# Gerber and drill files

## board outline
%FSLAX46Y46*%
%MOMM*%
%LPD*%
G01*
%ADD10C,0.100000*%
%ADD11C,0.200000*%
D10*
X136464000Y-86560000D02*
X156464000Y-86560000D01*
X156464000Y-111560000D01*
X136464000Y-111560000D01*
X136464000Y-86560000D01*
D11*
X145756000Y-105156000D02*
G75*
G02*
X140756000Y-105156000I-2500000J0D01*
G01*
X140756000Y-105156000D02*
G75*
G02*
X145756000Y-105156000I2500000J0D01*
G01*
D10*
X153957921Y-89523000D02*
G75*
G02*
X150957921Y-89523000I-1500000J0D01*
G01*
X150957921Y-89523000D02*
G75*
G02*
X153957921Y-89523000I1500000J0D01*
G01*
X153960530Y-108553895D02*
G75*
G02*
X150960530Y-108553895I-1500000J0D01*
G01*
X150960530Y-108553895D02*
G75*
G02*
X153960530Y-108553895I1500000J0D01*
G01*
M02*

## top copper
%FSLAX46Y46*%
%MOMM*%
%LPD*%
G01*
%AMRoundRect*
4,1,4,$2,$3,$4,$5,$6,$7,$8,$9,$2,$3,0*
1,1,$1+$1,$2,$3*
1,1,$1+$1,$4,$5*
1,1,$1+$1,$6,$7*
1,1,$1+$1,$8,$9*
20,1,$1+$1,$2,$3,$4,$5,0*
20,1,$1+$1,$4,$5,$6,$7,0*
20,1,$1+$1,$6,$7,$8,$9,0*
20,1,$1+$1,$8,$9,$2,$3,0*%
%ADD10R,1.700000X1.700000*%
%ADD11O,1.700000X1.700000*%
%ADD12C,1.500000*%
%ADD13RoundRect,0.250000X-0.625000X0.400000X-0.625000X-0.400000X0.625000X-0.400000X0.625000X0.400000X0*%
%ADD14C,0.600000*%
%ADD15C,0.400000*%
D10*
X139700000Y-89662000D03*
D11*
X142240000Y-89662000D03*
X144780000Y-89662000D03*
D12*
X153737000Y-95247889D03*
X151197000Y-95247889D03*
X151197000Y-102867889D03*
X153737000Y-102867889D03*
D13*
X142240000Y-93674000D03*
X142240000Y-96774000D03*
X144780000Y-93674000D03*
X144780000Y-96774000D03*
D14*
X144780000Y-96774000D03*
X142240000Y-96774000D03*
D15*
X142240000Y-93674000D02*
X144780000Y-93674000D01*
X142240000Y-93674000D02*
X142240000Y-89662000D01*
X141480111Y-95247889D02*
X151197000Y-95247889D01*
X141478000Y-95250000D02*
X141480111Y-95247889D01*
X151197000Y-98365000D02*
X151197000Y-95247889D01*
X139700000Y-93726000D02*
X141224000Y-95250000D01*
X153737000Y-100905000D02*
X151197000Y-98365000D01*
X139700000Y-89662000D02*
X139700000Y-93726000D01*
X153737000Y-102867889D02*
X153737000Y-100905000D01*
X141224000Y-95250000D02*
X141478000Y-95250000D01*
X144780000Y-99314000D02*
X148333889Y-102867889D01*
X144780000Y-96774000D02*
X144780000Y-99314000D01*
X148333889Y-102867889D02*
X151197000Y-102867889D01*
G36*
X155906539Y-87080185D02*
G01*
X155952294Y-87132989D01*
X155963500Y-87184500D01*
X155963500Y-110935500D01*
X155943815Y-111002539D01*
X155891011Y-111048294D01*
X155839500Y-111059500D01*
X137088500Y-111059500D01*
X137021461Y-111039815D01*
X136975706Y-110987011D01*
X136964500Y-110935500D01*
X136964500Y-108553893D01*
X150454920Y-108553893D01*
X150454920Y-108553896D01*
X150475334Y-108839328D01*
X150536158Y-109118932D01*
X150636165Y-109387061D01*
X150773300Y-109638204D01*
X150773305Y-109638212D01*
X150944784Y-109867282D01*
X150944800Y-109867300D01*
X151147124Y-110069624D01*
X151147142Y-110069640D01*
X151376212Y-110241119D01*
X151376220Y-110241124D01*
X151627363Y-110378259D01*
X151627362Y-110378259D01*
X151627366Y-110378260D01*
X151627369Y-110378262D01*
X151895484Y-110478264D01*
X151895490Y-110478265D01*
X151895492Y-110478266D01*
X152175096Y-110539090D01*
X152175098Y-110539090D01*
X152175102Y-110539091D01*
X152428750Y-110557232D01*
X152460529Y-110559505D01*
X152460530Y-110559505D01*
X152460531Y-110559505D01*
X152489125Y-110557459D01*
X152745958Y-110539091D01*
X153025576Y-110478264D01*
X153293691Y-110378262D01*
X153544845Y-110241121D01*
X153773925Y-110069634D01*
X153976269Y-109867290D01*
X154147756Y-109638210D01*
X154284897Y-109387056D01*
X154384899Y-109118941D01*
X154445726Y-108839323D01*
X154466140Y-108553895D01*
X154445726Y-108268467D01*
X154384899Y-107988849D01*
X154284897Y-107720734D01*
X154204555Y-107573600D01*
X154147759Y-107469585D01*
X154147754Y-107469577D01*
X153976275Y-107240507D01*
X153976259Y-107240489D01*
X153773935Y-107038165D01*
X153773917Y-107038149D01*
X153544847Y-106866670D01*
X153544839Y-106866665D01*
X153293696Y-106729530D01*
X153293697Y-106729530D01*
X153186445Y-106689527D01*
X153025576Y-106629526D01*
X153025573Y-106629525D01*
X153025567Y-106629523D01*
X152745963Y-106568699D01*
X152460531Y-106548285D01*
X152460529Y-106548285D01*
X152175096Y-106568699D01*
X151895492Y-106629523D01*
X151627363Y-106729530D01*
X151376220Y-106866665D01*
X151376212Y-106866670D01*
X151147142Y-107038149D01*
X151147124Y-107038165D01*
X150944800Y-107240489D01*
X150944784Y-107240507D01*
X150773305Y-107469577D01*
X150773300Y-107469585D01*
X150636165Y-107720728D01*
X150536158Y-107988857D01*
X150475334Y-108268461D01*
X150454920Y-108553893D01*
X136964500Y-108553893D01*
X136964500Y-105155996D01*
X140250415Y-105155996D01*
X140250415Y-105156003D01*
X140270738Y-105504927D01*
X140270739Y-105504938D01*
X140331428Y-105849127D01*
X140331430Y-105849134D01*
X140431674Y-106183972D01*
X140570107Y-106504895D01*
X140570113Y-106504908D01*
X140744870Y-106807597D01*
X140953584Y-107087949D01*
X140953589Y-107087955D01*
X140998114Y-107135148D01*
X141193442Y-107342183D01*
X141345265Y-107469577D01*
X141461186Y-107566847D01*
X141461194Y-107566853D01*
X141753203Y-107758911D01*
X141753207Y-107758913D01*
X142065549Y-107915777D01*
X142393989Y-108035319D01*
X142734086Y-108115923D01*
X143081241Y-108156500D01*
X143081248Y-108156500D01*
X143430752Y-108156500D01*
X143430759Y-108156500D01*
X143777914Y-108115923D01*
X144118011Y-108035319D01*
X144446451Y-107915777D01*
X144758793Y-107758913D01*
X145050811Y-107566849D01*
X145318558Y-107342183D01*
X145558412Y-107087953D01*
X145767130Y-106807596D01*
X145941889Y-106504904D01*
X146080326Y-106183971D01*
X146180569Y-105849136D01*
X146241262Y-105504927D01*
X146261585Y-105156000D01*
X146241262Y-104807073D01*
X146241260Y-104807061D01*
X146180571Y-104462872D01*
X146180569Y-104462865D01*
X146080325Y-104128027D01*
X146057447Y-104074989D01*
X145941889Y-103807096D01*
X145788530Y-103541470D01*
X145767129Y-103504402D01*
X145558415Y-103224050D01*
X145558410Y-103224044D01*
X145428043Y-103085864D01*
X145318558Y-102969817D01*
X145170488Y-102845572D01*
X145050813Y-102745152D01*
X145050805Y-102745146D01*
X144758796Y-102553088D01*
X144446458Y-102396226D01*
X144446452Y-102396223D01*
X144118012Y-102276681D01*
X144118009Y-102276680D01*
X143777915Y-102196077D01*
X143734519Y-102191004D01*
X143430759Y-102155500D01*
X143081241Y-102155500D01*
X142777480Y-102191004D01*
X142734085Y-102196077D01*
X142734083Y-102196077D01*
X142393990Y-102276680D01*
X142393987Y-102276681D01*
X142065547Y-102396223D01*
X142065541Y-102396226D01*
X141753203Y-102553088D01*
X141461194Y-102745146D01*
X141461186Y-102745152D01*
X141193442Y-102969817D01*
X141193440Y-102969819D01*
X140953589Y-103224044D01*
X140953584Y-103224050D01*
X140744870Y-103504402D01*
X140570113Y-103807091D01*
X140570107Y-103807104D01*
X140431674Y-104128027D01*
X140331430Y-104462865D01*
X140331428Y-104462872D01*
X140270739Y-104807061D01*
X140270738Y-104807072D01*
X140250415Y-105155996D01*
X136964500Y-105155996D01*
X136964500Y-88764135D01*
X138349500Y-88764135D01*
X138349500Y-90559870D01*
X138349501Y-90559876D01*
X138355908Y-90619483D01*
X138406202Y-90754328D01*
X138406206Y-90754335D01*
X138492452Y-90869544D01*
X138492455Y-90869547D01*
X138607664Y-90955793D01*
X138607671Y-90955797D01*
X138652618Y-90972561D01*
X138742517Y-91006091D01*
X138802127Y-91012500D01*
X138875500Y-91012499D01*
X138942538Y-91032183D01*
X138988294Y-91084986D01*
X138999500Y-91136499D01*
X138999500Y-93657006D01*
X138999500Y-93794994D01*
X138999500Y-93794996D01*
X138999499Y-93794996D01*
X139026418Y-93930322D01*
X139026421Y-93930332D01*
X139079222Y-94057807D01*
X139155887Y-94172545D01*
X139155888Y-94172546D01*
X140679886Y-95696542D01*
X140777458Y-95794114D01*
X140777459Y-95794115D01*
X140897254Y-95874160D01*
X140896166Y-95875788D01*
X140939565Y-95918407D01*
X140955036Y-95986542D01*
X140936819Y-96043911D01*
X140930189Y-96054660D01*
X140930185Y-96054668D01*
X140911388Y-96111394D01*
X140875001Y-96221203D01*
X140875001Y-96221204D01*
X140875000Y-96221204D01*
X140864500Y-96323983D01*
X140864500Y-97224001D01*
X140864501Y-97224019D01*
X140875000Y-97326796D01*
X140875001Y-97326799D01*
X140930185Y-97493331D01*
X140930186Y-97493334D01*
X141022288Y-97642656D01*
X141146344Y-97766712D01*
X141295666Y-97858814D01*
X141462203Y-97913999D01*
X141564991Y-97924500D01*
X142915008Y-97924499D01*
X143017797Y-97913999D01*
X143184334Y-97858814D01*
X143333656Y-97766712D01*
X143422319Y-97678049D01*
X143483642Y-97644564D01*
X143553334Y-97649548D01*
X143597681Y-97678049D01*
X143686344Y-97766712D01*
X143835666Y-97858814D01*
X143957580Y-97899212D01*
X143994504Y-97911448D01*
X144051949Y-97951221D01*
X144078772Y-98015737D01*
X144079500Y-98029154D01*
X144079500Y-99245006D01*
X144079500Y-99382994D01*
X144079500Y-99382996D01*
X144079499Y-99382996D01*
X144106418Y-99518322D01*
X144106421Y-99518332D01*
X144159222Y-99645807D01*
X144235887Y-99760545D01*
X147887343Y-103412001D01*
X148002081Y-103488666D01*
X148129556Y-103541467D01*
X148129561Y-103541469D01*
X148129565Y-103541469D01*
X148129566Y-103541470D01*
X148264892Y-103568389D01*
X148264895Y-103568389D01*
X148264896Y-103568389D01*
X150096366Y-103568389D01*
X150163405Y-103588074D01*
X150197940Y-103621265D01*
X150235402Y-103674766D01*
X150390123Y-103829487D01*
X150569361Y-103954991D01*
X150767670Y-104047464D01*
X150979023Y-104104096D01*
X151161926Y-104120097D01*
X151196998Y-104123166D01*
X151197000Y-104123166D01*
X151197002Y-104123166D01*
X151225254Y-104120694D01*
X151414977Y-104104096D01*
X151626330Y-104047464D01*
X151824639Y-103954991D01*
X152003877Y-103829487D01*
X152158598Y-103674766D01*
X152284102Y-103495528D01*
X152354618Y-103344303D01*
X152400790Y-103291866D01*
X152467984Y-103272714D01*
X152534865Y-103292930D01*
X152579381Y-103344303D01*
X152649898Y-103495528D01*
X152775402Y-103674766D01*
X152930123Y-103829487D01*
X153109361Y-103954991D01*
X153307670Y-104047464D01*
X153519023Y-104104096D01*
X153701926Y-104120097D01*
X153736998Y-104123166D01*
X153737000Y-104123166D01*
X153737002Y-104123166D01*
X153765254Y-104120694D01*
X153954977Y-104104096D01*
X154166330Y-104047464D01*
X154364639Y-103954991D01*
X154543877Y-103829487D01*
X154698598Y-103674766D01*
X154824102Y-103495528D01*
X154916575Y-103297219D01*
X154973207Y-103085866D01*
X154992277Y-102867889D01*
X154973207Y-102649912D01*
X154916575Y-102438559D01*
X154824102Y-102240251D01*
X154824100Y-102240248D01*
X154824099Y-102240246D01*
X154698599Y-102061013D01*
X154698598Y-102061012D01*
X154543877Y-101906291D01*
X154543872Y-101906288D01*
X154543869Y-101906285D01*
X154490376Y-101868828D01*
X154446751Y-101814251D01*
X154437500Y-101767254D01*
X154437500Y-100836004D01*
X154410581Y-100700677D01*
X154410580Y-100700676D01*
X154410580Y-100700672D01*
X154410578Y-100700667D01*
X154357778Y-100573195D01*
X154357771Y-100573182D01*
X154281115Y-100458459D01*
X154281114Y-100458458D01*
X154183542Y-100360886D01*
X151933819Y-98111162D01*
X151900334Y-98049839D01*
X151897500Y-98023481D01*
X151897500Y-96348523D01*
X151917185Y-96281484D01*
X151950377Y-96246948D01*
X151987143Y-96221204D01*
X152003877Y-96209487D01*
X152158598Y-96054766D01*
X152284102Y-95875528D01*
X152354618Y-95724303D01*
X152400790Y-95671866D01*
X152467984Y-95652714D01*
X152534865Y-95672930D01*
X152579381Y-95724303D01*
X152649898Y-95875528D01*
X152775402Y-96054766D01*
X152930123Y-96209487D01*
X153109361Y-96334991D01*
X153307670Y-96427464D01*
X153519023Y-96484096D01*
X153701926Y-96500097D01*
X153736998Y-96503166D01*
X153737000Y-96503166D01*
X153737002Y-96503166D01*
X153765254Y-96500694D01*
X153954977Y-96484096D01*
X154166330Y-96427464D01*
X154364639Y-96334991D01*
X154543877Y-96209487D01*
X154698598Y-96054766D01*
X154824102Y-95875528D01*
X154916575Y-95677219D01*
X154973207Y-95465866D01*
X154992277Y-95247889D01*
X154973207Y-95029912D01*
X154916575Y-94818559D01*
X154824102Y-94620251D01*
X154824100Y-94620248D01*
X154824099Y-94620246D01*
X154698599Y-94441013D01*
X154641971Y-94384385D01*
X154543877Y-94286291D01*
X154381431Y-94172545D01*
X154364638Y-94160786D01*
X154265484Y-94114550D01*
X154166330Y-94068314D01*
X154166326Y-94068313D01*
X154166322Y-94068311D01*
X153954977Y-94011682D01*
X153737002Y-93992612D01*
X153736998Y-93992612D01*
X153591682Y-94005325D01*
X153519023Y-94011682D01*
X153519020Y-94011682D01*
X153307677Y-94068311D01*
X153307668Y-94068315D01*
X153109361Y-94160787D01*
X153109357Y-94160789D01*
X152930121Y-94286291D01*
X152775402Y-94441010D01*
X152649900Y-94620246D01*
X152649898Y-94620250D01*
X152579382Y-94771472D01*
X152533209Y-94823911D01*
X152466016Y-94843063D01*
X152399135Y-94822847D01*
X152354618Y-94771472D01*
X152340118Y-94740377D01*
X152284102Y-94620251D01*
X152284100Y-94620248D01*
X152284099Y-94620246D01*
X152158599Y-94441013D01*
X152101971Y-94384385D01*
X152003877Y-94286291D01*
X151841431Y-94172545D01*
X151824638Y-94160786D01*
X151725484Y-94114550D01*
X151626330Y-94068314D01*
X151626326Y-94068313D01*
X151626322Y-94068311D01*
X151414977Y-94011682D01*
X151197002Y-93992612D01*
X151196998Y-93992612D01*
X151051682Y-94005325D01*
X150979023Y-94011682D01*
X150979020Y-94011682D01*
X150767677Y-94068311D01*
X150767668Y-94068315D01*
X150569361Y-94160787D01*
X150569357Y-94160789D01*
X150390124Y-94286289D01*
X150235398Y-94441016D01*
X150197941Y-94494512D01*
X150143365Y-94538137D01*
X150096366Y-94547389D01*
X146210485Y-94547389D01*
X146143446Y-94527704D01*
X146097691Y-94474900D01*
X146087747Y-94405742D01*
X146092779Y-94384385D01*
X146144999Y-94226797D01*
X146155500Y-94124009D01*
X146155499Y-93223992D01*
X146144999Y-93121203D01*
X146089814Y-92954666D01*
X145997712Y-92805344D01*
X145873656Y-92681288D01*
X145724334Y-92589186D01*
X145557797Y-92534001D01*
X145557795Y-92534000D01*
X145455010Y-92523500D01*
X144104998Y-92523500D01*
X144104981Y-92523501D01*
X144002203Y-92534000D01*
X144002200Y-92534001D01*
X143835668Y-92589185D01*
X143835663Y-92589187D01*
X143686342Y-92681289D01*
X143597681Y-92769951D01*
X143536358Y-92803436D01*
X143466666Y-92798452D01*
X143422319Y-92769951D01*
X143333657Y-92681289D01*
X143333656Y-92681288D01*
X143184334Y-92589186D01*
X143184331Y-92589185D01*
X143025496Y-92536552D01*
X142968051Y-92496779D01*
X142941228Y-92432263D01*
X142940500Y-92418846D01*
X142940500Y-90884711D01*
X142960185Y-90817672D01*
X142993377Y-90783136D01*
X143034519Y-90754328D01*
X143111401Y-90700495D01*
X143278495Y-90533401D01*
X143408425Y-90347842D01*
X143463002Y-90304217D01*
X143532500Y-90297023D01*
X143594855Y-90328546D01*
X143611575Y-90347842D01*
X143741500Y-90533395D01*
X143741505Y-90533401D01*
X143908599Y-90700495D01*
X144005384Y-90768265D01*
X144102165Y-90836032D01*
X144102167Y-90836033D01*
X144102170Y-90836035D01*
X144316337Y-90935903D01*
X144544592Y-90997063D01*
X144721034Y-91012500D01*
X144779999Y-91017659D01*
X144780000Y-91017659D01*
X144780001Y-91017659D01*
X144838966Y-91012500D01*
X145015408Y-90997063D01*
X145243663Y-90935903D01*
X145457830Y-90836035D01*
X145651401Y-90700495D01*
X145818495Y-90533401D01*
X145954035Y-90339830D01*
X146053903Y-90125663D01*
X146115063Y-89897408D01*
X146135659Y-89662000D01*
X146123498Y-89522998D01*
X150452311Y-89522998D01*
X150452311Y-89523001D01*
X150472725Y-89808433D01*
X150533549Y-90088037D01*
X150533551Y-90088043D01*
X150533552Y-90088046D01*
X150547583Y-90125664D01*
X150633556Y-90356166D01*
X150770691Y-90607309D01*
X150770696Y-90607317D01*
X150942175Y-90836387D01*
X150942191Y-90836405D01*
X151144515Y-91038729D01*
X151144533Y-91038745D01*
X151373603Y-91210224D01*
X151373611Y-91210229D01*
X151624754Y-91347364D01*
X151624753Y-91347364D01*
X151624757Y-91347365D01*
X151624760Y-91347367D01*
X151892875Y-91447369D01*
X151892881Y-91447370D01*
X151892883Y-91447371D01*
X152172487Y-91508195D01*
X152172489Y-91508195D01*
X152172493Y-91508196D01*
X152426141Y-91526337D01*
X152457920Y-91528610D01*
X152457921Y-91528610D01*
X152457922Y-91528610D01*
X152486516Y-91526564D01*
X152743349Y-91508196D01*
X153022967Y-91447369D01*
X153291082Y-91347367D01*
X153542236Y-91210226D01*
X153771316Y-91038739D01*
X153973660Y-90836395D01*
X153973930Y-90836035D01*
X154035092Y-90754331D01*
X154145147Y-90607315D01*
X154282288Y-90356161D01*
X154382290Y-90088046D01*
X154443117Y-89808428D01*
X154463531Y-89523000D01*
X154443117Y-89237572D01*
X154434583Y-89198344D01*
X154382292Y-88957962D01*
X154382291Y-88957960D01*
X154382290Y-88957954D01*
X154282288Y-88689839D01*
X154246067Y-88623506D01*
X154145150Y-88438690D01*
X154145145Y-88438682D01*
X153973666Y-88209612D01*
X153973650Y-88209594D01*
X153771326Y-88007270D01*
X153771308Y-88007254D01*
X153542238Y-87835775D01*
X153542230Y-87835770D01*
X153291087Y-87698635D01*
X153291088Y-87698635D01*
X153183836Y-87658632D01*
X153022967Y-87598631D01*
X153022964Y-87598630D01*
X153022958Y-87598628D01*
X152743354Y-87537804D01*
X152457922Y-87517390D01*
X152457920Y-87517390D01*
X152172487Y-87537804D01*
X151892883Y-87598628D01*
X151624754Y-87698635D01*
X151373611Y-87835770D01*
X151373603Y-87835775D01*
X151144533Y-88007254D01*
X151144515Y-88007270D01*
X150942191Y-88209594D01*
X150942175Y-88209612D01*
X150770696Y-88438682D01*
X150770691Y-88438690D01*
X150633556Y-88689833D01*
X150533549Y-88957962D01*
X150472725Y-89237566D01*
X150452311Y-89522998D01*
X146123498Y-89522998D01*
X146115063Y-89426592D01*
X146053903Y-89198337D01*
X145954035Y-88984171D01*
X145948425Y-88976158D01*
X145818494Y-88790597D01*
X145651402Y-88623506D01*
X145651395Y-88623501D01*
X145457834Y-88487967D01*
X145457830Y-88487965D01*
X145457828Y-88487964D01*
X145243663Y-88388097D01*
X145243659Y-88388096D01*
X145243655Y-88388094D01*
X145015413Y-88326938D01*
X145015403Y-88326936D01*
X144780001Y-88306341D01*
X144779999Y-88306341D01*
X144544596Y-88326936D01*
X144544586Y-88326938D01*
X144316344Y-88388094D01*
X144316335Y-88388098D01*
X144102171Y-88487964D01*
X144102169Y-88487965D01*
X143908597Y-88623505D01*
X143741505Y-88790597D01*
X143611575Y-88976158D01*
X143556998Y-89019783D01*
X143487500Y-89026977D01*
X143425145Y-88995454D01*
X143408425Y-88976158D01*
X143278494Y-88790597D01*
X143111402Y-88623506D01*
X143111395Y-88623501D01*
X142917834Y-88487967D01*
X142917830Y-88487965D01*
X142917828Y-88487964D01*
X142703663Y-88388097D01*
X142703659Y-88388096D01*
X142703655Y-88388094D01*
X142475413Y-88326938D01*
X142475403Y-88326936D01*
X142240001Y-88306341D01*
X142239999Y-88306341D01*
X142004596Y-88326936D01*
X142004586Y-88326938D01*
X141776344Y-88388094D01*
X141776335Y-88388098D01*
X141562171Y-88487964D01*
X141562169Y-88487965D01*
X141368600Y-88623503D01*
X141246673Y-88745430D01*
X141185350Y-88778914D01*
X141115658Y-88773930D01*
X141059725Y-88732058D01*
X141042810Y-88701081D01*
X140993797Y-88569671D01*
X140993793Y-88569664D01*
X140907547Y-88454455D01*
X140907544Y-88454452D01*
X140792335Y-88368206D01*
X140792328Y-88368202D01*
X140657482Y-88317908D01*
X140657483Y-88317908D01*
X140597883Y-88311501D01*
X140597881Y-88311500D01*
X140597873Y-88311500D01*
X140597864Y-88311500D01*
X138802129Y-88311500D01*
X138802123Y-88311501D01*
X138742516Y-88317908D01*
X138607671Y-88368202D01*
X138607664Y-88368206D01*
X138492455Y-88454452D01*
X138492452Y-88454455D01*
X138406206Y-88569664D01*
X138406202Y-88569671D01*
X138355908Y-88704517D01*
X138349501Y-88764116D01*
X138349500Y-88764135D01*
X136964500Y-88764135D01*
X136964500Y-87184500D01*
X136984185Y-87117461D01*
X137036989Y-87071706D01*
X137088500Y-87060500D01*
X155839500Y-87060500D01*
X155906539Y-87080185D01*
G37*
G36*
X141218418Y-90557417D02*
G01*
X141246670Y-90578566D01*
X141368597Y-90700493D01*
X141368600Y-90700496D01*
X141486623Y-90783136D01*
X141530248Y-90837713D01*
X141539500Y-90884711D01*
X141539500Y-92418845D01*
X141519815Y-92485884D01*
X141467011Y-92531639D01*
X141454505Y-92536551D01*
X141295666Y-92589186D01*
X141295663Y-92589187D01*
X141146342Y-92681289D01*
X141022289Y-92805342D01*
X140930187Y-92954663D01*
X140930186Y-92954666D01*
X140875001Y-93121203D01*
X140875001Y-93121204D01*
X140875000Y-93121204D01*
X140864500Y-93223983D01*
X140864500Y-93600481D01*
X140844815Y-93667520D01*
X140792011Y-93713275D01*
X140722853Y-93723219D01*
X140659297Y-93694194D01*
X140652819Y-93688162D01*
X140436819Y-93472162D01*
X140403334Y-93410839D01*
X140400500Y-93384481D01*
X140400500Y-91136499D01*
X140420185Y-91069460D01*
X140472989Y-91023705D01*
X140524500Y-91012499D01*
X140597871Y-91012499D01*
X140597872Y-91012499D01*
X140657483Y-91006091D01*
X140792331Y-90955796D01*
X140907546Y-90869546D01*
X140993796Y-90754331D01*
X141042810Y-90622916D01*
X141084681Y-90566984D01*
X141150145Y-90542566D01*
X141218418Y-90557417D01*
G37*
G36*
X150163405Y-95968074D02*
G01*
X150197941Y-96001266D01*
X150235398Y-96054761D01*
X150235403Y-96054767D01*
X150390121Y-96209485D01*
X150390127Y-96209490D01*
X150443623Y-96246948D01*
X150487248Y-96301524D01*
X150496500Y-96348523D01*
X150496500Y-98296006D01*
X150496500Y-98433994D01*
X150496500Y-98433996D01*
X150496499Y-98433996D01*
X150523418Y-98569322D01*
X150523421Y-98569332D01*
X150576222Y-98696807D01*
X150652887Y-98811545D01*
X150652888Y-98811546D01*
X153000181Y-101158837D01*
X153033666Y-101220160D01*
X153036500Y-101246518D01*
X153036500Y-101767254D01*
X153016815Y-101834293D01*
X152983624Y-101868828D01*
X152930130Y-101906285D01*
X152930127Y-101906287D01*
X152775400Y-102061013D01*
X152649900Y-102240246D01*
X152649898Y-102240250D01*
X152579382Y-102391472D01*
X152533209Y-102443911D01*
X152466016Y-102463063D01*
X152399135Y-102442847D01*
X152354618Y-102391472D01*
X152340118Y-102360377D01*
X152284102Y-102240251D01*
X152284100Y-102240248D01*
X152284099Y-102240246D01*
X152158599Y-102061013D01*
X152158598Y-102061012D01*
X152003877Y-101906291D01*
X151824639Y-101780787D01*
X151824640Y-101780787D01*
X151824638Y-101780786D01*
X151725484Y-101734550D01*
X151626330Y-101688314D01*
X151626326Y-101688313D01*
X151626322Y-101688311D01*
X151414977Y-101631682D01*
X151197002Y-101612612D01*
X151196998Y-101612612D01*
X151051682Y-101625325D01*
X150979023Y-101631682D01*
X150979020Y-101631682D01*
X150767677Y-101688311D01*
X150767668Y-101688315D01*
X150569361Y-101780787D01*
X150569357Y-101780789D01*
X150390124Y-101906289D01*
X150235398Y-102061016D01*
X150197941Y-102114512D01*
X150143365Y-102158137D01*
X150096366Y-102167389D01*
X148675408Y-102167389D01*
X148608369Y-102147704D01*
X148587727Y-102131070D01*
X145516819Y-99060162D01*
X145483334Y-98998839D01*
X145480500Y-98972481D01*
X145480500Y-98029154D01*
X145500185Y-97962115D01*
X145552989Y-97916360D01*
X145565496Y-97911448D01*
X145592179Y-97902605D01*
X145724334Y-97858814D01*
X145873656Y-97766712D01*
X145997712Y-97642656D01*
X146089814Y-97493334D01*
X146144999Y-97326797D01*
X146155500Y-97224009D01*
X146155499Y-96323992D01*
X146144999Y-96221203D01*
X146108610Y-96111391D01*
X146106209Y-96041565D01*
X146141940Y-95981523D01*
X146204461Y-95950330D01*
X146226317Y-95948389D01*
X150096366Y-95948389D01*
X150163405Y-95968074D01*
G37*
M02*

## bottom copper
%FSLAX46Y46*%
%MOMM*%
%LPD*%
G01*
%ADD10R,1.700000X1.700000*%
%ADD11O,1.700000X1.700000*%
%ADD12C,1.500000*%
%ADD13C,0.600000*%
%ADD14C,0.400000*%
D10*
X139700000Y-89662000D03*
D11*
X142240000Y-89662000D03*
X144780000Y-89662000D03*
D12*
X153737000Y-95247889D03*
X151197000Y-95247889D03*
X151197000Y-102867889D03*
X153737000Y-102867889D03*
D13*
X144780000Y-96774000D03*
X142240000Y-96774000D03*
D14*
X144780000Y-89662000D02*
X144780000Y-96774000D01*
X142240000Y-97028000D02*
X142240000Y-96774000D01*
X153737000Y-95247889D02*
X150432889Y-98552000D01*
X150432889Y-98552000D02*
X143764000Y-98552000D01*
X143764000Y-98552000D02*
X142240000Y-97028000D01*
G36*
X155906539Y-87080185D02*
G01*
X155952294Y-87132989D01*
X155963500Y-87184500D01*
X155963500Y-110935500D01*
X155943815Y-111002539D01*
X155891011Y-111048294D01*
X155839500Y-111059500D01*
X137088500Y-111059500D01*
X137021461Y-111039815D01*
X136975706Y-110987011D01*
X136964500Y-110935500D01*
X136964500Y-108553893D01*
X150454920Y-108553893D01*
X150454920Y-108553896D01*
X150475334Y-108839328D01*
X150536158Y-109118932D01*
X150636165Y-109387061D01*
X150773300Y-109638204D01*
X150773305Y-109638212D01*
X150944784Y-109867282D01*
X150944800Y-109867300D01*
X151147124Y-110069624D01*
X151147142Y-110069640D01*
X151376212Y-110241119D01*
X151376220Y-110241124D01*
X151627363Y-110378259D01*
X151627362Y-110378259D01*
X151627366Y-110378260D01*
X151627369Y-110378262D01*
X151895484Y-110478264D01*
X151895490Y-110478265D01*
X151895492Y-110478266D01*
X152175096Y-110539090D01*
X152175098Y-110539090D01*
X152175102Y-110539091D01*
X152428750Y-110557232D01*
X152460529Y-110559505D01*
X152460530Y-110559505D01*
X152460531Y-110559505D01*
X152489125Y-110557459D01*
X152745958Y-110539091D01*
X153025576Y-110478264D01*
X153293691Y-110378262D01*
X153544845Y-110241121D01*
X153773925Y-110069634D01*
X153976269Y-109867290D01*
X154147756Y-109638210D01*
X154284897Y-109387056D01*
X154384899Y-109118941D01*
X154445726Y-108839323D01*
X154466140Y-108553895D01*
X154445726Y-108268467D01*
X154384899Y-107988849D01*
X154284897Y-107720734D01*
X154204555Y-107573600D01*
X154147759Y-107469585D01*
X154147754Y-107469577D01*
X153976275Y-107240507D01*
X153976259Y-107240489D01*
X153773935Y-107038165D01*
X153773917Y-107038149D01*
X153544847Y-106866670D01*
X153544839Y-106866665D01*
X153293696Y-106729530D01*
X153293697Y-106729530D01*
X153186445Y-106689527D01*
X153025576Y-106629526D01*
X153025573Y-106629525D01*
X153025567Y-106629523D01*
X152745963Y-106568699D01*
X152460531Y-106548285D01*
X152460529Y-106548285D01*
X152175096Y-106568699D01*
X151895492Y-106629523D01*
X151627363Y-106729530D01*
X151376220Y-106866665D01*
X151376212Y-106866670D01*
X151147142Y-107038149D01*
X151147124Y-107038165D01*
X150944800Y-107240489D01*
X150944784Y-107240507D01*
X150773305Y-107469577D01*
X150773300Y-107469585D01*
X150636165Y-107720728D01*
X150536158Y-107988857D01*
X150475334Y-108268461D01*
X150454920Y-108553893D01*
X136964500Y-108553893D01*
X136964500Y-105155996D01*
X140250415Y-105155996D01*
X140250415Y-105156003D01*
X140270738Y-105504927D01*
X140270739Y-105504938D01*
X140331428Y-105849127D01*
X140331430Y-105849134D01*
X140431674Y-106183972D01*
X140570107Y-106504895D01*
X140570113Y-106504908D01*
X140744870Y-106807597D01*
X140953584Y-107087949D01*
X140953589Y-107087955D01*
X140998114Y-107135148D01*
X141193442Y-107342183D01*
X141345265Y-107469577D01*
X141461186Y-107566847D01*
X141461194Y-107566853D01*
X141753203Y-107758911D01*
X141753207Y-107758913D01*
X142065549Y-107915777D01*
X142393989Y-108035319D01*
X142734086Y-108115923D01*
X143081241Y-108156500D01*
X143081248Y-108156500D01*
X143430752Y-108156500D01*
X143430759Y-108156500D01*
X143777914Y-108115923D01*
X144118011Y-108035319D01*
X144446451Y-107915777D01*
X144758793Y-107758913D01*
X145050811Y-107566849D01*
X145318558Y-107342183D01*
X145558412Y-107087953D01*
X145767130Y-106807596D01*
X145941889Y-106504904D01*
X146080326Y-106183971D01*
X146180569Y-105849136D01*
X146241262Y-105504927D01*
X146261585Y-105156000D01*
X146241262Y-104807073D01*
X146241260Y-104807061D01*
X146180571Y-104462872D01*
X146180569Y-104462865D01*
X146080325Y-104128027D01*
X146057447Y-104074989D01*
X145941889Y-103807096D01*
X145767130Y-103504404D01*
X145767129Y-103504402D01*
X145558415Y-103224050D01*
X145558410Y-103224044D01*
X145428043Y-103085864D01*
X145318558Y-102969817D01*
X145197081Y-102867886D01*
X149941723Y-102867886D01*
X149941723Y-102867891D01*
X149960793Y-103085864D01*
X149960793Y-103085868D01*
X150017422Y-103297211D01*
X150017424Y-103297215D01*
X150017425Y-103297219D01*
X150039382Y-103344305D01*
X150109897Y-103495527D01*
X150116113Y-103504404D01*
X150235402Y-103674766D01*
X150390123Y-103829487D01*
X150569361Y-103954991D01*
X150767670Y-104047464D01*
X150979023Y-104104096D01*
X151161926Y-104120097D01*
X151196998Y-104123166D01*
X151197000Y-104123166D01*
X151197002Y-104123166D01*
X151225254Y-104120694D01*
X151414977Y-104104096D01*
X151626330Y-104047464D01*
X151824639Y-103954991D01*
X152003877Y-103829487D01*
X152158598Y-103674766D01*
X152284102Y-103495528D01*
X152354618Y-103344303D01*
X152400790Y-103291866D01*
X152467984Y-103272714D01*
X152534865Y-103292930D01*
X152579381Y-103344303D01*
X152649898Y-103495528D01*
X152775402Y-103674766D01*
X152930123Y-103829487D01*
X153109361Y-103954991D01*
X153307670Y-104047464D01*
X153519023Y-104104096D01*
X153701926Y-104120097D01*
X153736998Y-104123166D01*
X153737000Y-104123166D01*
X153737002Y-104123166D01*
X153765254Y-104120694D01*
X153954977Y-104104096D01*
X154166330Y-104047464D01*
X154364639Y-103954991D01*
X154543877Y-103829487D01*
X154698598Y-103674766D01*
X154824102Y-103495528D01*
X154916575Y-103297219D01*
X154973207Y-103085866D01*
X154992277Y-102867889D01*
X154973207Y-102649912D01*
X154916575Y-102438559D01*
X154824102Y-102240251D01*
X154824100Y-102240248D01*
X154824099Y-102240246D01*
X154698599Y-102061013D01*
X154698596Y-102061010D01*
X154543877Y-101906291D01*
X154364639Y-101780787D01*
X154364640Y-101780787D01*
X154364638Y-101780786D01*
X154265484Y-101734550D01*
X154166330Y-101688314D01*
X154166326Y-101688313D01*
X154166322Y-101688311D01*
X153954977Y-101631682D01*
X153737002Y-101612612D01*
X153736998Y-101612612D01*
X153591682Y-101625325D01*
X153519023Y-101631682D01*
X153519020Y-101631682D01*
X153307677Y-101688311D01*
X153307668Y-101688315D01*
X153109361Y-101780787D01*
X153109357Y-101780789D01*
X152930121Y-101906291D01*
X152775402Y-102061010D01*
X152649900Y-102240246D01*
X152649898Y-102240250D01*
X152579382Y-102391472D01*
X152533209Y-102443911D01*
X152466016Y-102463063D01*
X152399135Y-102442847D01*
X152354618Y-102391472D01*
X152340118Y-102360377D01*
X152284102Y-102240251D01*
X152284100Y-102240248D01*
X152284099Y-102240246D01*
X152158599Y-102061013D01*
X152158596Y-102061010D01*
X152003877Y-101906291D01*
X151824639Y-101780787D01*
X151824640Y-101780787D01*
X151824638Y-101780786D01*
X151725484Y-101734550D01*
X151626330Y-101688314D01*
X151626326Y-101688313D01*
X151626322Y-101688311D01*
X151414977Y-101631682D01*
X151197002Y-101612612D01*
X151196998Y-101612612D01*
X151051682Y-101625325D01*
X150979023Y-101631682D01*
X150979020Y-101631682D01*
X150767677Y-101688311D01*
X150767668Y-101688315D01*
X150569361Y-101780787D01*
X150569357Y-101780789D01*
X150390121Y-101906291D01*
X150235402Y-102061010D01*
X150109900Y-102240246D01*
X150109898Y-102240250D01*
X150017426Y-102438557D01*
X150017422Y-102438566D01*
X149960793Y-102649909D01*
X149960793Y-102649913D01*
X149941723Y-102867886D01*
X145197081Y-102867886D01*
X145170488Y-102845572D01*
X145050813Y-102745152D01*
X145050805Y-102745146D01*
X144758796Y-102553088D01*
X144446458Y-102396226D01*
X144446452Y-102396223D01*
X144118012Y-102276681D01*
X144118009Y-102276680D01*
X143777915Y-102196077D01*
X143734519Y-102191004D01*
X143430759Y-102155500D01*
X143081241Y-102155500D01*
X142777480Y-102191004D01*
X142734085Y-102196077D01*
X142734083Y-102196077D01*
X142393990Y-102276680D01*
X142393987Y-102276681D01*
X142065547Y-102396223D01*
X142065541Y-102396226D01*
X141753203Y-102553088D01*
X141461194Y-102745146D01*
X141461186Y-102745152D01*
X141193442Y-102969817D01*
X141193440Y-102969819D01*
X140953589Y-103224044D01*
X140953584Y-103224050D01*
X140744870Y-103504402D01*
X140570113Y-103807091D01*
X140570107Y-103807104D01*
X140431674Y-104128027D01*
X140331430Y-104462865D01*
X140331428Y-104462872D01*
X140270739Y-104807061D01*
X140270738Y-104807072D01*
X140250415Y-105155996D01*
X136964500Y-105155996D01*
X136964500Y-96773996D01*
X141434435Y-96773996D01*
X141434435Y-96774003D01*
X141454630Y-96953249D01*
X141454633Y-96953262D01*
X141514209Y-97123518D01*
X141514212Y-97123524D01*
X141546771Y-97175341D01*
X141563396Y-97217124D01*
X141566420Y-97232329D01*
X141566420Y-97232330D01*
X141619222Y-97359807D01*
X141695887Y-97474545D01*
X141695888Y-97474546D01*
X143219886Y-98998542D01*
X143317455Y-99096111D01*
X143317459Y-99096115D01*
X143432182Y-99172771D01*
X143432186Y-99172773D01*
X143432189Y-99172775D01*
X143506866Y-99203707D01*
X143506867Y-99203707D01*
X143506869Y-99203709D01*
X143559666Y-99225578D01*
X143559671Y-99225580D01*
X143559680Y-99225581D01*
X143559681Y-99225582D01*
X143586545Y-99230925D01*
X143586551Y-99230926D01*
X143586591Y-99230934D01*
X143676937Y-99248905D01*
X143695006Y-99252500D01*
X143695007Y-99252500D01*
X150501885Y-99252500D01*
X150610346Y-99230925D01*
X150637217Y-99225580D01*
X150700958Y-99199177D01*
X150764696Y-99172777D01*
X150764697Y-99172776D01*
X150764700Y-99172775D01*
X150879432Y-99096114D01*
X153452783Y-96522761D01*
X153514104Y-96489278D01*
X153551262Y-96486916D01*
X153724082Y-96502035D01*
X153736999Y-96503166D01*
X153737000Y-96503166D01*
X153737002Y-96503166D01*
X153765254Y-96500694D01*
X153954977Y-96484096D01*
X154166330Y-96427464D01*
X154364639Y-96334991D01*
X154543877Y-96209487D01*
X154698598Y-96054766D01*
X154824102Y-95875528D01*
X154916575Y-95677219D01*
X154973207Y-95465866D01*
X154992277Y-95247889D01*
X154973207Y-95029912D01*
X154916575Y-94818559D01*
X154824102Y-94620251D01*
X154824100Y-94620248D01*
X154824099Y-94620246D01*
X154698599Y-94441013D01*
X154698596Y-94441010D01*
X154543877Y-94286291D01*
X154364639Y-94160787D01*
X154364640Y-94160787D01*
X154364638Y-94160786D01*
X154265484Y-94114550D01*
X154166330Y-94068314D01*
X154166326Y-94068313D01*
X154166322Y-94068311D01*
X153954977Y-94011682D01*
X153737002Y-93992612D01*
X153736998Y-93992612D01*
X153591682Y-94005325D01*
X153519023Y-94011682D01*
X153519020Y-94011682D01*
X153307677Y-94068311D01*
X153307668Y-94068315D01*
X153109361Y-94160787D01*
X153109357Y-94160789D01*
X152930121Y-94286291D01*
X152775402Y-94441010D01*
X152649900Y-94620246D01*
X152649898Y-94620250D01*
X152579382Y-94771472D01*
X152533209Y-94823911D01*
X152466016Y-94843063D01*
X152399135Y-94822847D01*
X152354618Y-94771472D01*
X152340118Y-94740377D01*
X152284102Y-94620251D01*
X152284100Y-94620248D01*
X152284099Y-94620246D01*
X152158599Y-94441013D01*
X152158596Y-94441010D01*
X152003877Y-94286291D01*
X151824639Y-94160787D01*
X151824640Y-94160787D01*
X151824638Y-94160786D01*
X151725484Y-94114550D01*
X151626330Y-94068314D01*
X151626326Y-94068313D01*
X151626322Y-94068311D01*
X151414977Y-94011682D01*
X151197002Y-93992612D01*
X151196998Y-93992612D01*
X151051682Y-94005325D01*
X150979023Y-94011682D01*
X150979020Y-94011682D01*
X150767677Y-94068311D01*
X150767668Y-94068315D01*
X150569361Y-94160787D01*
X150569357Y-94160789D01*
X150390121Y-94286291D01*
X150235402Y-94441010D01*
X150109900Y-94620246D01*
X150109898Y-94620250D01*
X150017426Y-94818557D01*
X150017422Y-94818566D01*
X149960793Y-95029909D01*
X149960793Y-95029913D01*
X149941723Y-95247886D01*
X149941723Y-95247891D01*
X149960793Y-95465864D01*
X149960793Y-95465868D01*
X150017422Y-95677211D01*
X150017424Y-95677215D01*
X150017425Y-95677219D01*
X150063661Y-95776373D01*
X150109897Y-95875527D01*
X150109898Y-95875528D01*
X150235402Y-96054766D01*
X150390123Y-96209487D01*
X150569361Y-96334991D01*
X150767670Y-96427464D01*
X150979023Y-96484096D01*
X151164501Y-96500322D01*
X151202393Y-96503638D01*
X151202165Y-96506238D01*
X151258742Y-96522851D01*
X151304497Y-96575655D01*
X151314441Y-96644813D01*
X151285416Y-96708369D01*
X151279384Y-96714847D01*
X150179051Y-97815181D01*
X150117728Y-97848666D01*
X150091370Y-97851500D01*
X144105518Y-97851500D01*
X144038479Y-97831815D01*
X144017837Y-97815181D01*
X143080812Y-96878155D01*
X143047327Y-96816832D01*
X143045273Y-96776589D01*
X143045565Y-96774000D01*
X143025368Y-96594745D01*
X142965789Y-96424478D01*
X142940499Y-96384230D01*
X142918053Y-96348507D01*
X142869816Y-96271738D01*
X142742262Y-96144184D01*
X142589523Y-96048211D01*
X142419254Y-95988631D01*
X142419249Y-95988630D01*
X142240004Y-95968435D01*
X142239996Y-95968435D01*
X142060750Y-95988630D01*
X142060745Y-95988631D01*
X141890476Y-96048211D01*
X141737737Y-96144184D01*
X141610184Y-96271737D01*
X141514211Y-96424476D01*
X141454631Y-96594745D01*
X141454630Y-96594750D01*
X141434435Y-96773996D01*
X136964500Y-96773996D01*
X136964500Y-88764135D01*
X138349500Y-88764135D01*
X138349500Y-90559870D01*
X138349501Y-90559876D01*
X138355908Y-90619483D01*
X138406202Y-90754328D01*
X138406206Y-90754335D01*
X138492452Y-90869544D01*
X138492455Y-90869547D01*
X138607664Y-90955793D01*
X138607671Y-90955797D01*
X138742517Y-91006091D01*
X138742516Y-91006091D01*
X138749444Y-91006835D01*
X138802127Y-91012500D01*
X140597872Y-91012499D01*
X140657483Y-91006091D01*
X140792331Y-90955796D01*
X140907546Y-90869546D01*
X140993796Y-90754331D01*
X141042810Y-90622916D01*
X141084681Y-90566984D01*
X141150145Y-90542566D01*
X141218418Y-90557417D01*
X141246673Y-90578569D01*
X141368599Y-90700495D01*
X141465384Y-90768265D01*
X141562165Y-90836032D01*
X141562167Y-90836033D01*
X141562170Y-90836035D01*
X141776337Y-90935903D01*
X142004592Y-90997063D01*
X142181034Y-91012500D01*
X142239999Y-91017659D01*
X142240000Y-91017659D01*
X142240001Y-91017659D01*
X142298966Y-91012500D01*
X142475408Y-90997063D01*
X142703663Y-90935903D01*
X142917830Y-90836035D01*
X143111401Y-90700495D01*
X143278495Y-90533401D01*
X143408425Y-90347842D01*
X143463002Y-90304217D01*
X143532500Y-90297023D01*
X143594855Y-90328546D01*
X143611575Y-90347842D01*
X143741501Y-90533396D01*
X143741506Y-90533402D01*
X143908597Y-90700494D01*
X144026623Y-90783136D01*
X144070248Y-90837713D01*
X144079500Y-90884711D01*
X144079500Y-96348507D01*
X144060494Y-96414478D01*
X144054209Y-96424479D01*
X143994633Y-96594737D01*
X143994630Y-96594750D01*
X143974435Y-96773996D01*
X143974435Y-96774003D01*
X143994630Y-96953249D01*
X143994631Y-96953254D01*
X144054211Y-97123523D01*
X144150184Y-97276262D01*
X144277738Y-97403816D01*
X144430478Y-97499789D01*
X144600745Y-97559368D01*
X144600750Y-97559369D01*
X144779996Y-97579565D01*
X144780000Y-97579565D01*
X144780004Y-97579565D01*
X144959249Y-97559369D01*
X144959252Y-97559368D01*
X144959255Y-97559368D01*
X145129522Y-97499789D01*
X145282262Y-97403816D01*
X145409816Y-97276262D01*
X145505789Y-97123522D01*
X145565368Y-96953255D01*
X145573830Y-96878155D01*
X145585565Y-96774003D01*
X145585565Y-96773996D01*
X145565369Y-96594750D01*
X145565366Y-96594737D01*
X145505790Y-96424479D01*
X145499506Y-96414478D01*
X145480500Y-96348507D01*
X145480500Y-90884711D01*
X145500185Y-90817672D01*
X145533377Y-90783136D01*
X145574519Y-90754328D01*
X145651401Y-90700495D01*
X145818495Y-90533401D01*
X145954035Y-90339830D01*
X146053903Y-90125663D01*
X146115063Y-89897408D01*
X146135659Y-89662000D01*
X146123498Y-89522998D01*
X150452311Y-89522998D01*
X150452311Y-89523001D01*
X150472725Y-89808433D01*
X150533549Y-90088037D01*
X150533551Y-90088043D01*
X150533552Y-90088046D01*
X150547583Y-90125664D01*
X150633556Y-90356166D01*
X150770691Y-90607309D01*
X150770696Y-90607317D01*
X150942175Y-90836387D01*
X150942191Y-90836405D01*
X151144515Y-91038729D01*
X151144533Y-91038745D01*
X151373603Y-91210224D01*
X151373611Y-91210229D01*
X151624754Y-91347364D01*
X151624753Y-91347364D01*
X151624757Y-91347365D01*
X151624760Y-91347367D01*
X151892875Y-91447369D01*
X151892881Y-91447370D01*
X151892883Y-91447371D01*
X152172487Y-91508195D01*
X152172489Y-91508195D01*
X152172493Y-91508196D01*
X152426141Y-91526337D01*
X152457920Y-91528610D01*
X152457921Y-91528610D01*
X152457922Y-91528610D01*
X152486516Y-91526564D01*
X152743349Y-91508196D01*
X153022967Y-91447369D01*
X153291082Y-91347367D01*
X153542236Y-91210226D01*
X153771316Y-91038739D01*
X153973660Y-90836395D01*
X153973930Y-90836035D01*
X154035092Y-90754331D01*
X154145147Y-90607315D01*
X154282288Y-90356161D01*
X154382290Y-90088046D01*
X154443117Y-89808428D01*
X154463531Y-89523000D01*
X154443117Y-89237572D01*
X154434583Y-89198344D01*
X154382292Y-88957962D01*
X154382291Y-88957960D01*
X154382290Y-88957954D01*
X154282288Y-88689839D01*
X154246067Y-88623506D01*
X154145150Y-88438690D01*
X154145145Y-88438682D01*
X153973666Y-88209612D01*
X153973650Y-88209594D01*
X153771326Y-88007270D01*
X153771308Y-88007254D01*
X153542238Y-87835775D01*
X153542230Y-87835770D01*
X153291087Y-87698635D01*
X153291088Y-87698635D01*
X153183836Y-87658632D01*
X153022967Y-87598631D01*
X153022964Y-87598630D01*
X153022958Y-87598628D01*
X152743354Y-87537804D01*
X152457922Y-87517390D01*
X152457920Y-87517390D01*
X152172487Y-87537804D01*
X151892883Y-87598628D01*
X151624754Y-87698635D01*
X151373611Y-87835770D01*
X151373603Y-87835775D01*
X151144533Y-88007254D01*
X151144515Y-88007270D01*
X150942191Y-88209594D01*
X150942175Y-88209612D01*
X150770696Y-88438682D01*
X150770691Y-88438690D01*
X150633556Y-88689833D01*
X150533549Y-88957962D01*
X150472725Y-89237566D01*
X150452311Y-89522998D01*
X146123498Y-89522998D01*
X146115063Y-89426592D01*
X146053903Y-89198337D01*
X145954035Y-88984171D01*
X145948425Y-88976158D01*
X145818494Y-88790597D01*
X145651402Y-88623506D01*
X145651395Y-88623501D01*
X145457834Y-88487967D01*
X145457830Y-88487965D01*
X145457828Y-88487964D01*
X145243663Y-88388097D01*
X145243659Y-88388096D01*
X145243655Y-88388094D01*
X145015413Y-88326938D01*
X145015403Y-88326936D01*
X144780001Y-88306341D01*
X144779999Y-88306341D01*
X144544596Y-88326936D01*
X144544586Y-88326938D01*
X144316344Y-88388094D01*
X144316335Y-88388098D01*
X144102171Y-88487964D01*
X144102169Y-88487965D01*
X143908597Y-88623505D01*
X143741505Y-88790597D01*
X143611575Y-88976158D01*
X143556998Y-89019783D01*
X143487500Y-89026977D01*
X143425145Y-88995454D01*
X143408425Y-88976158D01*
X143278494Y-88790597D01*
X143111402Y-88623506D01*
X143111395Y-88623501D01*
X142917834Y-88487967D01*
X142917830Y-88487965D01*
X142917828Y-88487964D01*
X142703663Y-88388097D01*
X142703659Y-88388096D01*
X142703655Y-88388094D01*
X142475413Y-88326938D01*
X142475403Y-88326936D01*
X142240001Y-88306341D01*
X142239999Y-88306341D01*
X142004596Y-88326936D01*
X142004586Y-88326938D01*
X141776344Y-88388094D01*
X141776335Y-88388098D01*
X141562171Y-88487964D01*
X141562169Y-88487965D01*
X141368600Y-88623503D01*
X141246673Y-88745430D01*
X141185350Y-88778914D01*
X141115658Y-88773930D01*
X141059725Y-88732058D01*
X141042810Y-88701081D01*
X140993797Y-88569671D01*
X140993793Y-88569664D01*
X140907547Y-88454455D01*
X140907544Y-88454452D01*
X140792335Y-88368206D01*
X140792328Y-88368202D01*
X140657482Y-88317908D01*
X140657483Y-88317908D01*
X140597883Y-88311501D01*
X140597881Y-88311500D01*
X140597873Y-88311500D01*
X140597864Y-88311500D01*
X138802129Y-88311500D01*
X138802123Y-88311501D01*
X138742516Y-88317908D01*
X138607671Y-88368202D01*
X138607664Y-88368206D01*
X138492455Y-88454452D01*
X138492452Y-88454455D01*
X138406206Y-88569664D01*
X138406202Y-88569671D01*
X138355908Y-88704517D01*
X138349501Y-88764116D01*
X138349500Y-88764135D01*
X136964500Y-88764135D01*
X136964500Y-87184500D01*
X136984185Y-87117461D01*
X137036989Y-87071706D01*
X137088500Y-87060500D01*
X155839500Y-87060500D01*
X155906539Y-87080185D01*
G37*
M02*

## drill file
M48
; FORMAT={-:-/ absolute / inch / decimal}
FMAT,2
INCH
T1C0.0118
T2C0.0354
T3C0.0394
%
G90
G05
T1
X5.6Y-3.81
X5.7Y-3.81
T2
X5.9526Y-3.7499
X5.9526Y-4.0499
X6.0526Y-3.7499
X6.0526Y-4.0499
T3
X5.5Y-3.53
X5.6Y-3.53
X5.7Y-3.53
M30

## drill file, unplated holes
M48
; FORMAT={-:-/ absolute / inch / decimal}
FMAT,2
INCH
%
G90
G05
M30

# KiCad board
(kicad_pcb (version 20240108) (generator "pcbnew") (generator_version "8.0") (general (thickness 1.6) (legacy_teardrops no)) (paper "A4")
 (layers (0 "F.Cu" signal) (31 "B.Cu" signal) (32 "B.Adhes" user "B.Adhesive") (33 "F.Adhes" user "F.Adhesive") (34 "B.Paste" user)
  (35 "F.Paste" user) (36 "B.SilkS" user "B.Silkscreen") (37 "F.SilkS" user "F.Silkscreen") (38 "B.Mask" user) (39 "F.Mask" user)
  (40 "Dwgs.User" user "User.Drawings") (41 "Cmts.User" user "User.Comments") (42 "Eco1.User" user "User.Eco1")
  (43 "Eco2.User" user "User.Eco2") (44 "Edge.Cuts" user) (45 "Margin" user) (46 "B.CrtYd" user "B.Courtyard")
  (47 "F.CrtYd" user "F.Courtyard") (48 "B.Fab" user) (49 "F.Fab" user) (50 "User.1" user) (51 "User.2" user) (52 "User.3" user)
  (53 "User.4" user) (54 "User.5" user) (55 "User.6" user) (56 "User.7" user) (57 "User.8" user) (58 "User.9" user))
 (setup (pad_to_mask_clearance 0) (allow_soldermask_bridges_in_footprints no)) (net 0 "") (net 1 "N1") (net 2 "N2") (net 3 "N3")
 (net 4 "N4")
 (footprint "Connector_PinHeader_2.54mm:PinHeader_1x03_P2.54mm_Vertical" (layer "F.Cu") (at 139.7 89.662 90)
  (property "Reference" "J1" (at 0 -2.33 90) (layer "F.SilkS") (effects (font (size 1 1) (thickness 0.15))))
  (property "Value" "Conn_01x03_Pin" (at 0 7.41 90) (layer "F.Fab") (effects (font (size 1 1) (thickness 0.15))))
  (pad "1" thru_hole rect (at 0 0 90) (size 1.7 1.7) (drill 1) (layers "*.Cu" "*.Mask") (remove_unused_layers no) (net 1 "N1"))
  (pad "2" thru_hole oval (at 0 2.54 90) (size 1.7 1.7) (drill 1) (layers "*.Cu" "*.Mask") (remove_unused_layers no) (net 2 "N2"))
  (pad "3" thru_hole oval (at 0 5.08 90) (size 1.7 1.7) (drill 1) (layers "*.Cu" "*.Mask") (remove_unused_layers no) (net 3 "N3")))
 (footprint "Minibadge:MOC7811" (layer "F.Cu") (at 152.467 99.565889)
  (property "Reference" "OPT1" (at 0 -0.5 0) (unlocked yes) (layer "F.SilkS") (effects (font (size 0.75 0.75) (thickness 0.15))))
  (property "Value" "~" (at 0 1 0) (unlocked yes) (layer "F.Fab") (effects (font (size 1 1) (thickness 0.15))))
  (fp_circle (center -0.009079 -10.042889) (end 1.490921 -10.042889) (stroke (width 0.1) (type default)) (fill none) (layer "Edge.Cuts"))
  (fp_circle (center -0.00647 8.988006) (end 1.49353 8.988006) (stroke (width 0.1) (type default)) (fill none) (layer "Edge.Cuts"))
  (pad "1" thru_hole circle (at 1.27 -4.318) (size 1.5 1.5) (drill 0.9) (layers "*.Cu" "*.Mask") (remove_unused_layers no) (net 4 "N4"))
  (pad "2" thru_hole circle (at -1.27 -4.318) (size 1.5 1.5) (drill 0.9) (layers "*.Cu" "*.Mask") (remove_unused_layers no) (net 1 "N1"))
  (pad "3" thru_hole circle (at -1.27 3.302) (size 1.5 1.5) (drill 0.9) (layers "*.Cu" "*.Mask") (remove_unused_layers no) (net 3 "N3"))
  (pad "4" thru_hole circle (at 1.27 3.302) (size 1.5 1.5) (drill 0.9) (layers "*.Cu" "*.Mask") (remove_unused_layers no) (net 1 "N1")))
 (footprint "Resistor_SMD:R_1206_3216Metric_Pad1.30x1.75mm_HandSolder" (layer "F.Cu") (at 142.24 95.224 -90)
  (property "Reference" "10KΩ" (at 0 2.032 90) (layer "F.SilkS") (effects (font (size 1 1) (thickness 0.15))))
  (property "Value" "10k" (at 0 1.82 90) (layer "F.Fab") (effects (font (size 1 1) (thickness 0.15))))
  (pad "1" smd roundrect (at -1.55 0 270) (size 1.3 1.75) (layers "F.Cu" "F.Paste" "F.Mask") (roundrect_rratio 0.192308) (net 2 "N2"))
  (pad "2" smd roundrect (at 1.55 0 270) (size 1.3 1.75) (layers "F.Cu" "F.Paste" "F.Mask") (roundrect_rratio 0.192308) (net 4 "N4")))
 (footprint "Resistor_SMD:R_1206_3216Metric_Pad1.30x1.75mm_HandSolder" (layer "F.Cu") (at 144.78 95.224 -90)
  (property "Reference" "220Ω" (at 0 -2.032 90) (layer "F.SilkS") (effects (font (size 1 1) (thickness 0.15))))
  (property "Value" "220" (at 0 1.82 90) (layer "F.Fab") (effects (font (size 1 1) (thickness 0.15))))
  (pad "1" smd roundrect (at -1.55 0 270) (size 1.3 1.75) (layers "F.Cu" "F.Paste" "F.Mask") (roundrect_rratio 0.192308) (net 2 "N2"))
  (pad "2" smd roundrect (at 1.55 0 270) (size 1.3 1.75) (layers "F.Cu" "F.Paste" "F.Mask") (roundrect_rratio 0.192308) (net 3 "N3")))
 (gr_rect (start 136.464 86.56) (end 156.464 111.56) (stroke (width 0.1) (type default)) (fill none) (layer "Edge.Cuts"))
 (gr_circle (center 143.256 105.156) (end 145.756 105.156) (stroke (width 0.2) (type default)) (fill none) (layer "Edge.Cuts"))
 (segment (start 142.24 93.674) (end 142.24 89.662) (width 0.4) (layer "F.Cu") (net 2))
 (segment (start 142.24 93.674) (end 144.78 93.674) (width 0.4) (layer "F.Cu") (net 2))
 (segment (start 141.480111 95.247889) (end 151.197 95.247889) (width 0.4) (layer "F.Cu") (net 1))
 (segment (start 141.478 95.25) (end 141.480111 95.247889) (width 0.4) (layer "F.Cu") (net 1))
 (segment (start 151.197 98.365) (end 151.197 95.247889) (width 0.4) (layer "F.Cu") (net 1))
 (segment (start 139.7 93.726) (end 141.224 95.25) (width 0.4) (layer "F.Cu") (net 1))
 (segment (start 153.737 100.905) (end 151.197 98.365) (width 0.4) (layer "F.Cu") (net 1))
 (segment (start 139.7 89.662) (end 139.7 93.726) (width 0.4) (layer "F.Cu") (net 1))
 (segment (start 153.737 102.867889) (end 153.737 100.905) (width 0.4) (layer "F.Cu") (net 1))
 (segment (start 141.224 95.25) (end 141.478 95.25) (width 0.4) (layer "F.Cu") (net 1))
 (segment (start 144.78 99.314) (end 148.333889 102.867889) (width 0.4) (layer "F.Cu") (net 3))
 (segment (start 144.78 96.774) (end 144.78 99.314) (width 0.4) (layer "F.Cu") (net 3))
 (segment (start 148.333889 102.867889) (end 151.197 102.867889) (width 0.4) (layer "F.Cu") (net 3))
 (via (at 144.78 96.774) (size 0.6) (drill 0.3) (layers "F.Cu" "B.Cu") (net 3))
 (segment (start 144.78 89.662) (end 144.78 96.774) (width 0.4) (layer "B.Cu") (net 3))
 (via (at 142.24 96.774) (size 0.6) (drill 0.3) (layers "F.Cu" "B.Cu") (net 4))
 (segment (start 142.24 97.028) (end 142.24 96.774) (width 0.4) (layer "B.Cu") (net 4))
 (segment (start 153.737 95.247889) (end 150.432889 98.552) (width 0.4) (layer "B.Cu") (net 4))
 (segment (start 150.432889 98.552) (end 143.764 98.552) (width 0.4) (layer "B.Cu") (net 4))
 (segment (start 143.764 98.552) (end 142.24 97.028) (width 0.4) (layer "B.Cu") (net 4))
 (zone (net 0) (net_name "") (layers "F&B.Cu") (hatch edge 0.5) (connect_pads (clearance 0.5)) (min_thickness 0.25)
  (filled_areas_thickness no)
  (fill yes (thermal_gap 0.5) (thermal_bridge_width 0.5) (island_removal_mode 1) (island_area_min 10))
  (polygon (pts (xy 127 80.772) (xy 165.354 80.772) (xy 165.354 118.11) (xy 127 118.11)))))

